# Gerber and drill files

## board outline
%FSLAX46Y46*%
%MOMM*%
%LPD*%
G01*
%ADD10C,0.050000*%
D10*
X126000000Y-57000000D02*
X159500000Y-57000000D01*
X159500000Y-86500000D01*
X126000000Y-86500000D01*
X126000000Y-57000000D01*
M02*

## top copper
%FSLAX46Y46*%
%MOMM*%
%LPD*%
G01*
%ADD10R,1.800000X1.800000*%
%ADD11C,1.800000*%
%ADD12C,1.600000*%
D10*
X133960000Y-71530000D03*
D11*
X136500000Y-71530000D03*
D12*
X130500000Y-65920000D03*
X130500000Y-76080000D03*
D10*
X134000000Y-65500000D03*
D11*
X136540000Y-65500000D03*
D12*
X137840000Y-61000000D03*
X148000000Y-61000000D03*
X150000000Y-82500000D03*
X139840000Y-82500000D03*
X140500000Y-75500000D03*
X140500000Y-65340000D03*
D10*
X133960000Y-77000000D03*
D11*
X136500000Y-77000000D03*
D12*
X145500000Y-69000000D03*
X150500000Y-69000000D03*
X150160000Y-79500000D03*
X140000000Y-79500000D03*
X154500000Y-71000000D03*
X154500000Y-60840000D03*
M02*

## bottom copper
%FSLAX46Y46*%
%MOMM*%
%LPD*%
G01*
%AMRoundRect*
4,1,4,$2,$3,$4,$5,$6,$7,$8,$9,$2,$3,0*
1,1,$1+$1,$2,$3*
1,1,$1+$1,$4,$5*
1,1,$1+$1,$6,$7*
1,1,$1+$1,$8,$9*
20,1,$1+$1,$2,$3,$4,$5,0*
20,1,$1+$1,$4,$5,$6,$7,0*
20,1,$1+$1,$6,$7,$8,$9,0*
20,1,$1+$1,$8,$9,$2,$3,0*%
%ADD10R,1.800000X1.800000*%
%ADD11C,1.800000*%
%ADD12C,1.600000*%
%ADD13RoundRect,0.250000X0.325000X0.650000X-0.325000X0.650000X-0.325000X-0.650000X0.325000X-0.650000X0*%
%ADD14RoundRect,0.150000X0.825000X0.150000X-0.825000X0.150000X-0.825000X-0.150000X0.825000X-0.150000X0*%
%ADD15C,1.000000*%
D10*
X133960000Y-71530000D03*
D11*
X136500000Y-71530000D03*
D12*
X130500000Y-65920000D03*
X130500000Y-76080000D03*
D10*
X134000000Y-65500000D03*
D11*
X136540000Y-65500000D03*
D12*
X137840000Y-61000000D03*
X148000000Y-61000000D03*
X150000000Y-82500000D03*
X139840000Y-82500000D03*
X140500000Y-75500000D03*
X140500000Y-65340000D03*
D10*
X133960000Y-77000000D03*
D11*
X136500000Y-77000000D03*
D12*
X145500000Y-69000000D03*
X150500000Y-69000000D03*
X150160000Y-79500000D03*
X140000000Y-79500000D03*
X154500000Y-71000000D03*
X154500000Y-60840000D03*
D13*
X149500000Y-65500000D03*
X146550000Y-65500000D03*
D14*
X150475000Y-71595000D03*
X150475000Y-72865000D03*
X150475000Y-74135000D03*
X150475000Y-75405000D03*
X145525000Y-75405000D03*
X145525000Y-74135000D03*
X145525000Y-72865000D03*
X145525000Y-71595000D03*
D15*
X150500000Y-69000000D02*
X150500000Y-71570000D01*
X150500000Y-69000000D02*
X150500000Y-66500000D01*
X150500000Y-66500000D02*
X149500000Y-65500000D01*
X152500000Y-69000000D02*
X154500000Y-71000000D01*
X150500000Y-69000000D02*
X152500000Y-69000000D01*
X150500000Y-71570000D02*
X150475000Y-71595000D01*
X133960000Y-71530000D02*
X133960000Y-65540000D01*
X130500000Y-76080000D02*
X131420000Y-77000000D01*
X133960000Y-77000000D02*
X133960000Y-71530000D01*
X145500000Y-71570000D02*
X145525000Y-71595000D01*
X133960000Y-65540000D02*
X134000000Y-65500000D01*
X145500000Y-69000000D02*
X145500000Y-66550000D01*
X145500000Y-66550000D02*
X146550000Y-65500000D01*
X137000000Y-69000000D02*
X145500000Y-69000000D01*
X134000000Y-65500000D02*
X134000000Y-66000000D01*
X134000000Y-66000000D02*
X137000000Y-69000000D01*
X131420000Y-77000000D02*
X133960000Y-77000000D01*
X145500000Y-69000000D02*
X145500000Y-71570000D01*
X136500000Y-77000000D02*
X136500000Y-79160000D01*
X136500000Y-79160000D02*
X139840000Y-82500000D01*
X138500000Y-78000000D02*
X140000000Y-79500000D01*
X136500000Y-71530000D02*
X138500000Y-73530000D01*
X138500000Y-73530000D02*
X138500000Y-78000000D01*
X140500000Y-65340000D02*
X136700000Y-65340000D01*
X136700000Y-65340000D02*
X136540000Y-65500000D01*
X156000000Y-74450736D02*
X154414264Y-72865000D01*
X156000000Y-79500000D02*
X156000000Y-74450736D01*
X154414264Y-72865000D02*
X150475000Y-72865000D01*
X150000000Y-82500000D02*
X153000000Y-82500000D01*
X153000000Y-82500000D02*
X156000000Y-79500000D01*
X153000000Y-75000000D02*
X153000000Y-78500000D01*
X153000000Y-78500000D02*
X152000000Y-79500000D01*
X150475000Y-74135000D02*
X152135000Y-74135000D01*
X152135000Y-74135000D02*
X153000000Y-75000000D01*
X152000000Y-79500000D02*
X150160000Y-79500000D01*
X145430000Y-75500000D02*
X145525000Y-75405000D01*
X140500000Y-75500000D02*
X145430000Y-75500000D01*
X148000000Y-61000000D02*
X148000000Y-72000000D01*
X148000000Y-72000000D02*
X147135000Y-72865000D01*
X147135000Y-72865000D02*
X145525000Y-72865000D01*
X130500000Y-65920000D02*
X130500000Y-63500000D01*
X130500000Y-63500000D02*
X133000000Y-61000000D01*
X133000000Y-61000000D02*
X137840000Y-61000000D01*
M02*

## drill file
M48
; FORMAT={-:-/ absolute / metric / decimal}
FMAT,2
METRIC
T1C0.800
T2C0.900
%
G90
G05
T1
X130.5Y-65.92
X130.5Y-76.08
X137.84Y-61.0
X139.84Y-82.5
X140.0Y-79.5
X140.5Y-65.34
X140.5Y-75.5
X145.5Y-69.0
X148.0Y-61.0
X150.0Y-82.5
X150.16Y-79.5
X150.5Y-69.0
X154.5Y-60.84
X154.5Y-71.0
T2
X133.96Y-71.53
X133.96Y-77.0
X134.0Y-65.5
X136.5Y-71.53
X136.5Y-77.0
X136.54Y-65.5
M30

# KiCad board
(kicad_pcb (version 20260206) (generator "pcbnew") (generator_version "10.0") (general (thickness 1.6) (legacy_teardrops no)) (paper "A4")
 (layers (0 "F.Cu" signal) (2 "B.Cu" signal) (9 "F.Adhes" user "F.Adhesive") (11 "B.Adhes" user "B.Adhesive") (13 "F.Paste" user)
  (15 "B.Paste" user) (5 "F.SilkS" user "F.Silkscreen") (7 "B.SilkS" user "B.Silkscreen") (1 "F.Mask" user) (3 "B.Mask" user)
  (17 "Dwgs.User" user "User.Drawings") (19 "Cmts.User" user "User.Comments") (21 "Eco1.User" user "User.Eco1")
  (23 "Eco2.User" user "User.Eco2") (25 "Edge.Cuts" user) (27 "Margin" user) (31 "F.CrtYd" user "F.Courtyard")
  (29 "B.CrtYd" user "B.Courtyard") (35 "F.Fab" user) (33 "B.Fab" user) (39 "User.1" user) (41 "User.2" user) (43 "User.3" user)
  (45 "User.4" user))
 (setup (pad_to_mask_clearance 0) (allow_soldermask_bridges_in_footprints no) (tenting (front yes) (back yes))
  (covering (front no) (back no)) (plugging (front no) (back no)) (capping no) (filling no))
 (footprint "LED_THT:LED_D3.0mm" (layer "F.Cu") (at 133.96 71.53)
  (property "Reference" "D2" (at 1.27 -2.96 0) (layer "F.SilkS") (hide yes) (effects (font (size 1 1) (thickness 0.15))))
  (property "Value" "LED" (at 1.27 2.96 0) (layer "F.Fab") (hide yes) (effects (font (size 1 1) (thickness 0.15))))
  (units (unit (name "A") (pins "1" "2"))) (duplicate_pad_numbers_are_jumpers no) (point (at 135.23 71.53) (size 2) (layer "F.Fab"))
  (pad "1" thru_hole rect (at 0 0) (size 1.8 1.8) (drill 0.9) (layers "*.Cu" "*.Mask") (remove_unused_layers no) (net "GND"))
  (pad "2" thru_hole circle (at 2.54 0) (size 1.8 1.8) (drill 0.9) (layers "*.Cu" "*.Mask") (remove_unused_layers no) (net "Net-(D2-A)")))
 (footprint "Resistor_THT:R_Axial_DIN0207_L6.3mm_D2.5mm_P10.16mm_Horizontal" (layer "F.Cu") (at 130.5 65.92 -90)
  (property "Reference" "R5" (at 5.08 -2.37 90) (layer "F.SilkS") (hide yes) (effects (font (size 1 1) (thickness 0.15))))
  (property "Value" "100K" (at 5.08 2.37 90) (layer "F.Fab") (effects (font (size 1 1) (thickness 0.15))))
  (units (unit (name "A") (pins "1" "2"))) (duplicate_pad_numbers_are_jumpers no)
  (pad "1" thru_hole circle (at 0 0 270) (size 1.6 1.6) (drill 0.8) (layers "*.Cu" "*.Mask") (remove_unused_layers no)
   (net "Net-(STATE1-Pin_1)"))
  (pad "2" thru_hole circle (at 10.16 0 270) (size 1.6 1.6) (drill 0.8) (layers "*.Cu" "*.Mask") (remove_unused_layers no) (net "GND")))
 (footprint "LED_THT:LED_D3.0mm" (layer "F.Cu") (at 134 65.5)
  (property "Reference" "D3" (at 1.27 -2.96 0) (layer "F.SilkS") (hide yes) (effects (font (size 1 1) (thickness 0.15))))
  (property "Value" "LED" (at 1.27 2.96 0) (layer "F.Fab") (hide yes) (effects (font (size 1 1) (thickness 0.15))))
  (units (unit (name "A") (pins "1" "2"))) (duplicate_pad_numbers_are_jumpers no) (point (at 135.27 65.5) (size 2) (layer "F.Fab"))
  (pad "1" thru_hole rect (at 0 0) (size 1.8 1.8) (drill 0.9) (layers "*.Cu" "*.Mask") (remove_unused_layers no) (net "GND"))
  (pad "2" thru_hole circle (at 2.54 0) (size 1.8 1.8) (drill 0.9) (layers "*.Cu" "*.Mask") (remove_unused_layers no) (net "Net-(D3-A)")))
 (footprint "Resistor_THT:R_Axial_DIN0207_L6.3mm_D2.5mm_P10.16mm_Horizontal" (layer "F.Cu") (at 137.84 61)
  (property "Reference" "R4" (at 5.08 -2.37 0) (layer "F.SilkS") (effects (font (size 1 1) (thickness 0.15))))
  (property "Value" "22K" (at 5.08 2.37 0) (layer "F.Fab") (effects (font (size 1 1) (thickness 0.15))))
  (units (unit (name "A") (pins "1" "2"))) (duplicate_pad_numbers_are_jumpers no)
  (pad "1" thru_hole circle (at 0 0) (size 1.6 1.6) (drill 0.8) (layers "*.Cu" "*.Mask") (remove_unused_layers no)
   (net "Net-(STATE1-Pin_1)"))
  (pad "2" thru_hole circle (at 10.16 0) (size 1.6 1.6) (drill 0.8) (layers "*.Cu" "*.Mask") (remove_unused_layers no) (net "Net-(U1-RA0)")))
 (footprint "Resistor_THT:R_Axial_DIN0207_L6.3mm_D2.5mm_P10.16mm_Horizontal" (layer "F.Cu") (at 150 82.5 180)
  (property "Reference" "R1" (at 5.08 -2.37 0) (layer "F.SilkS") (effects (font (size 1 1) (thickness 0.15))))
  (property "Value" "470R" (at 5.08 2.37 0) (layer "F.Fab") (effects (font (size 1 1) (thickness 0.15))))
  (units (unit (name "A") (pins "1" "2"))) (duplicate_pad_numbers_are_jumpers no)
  (pad "1" thru_hole circle (at 0 0 180) (size 1.6 1.6) (drill 0.8) (layers "*.Cu" "*.Mask") (remove_unused_layers no) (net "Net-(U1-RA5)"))
  (pad "2" thru_hole circle (at 10.16 0 180) (size 1.6 1.6) (drill 0.8) (layers "*.Cu" "*.Mask") (remove_unused_layers no)
   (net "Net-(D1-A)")))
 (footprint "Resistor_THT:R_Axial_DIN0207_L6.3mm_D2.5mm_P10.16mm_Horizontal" (layer "F.Cu") (at 140.5 75.5 90)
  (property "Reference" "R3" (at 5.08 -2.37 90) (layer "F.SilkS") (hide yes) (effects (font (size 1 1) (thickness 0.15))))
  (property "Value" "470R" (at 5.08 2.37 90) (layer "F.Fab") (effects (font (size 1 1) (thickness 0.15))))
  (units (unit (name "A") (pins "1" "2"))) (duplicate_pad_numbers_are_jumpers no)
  (pad "1" thru_hole circle (at 0 0 90) (size 1.6 1.6) (drill 0.8) (layers "*.Cu" "*.Mask") (remove_unused_layers no) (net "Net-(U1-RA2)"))
  (pad "2" thru_hole circle (at 10.16 0 90) (size 1.6 1.6) (drill 0.8) (layers "*.Cu" "*.Mask") (remove_unused_layers no) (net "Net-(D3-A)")))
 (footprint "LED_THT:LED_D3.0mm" (layer "F.Cu") (at 133.96 77)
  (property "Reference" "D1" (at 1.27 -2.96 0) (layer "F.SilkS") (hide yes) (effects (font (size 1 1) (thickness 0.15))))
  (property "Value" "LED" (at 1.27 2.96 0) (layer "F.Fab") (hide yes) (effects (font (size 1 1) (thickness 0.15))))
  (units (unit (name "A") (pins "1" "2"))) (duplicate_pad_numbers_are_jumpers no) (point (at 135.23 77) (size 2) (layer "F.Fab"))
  (pad "1" thru_hole rect (at 0 0) (size 1.8 1.8) (drill 0.9) (layers "*.Cu" "*.Mask") (remove_unused_layers no) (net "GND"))
  (pad "2" thru_hole circle (at 2.54 0) (size 1.8 1.8) (drill 0.9) (layers "*.Cu" "*.Mask") (remove_unused_layers no) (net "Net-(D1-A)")))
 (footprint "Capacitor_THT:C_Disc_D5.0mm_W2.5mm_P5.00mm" (layer "F.Cu") (at 145.5 69)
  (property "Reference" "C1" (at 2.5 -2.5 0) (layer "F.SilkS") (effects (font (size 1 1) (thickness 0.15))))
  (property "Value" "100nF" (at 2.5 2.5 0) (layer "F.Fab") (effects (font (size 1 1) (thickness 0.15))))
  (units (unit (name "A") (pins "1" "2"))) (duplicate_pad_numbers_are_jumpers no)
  (pad "1" thru_hole circle (at 0 0) (size 1.6 1.6) (drill 0.8) (layers "*.Cu" "*.Mask") (remove_unused_layers no) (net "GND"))
  (pad "2" thru_hole circle (at 5 0) (size 1.6 1.6) (drill 0.8) (layers "*.Cu" "*.Mask") (remove_unused_layers no) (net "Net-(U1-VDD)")))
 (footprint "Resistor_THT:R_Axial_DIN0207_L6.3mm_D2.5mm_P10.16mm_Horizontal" (layer "F.Cu") (at 150.16 79.5 180)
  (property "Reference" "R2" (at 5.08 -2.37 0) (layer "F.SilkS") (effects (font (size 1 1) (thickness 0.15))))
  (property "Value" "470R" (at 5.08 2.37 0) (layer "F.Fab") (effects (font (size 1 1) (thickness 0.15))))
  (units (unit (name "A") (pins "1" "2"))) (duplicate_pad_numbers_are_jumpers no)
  (pad "1" thru_hole circle (at 0 0 180) (size 1.6 1.6) (drill 0.8) (layers "*.Cu" "*.Mask") (remove_unused_layers no) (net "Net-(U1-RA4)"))
  (pad "2" thru_hole circle (at 10.16 0 180) (size 1.6 1.6) (drill 0.8) (layers "*.Cu" "*.Mask") (remove_unused_layers no)
   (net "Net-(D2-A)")))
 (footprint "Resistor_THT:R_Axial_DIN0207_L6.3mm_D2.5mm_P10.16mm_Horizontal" (layer "F.Cu") (at 154.5 71 90)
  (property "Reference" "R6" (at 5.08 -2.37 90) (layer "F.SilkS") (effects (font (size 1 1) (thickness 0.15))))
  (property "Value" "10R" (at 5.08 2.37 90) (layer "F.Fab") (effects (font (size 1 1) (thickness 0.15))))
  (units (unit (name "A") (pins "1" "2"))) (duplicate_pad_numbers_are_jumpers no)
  (pad "1" thru_hole circle (at 0 0 90) (size 1.6 1.6) (drill 0.8) (layers "*.Cu" "*.Mask") (remove_unused_layers no) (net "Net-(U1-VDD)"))
  (pad "2" thru_hole circle (at 10.16 0 90) (size 1.6 1.6) (drill 0.8) (layers "*.Cu" "*.Mask") (remove_unused_layers no) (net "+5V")))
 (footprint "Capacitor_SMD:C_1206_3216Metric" (layer "B.Cu") (at 148.025 65.5 180)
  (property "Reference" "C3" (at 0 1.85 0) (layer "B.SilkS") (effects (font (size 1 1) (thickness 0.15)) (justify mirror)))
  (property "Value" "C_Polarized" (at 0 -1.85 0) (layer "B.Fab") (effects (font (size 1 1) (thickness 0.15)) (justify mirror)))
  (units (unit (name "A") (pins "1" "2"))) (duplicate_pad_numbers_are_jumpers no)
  (pad "1" smd roundrect (at -1.475 0 180) (size 1.15 1.8) (layers "B.Cu" "B.Mask" "B.Paste") (roundrect_rratio 0.217391)
   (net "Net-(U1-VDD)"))
  (pad "2" smd roundrect (at 1.475 0 180) (size 1.15 1.8) (layers "B.Cu" "B.Mask" "B.Paste") (roundrect_rratio 0.217391) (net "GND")))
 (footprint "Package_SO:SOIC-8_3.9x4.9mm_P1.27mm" (layer "B.Cu") (at 148 73.5 180)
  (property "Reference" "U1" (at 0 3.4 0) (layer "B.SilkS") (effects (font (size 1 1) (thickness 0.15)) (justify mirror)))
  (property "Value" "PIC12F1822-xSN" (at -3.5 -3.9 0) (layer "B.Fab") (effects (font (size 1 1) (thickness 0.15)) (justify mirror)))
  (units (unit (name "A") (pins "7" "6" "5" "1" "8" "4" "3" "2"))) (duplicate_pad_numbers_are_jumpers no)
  (pad "1" smd roundrect (at -2.475 1.905 180) (size 1.95 0.6) (layers "B.Cu" "B.Mask" "B.Paste") (roundrect_rratio 0.25)
   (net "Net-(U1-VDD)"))
  (pad "2" smd roundrect (at -2.475 0.635 180) (size 1.95 0.6) (layers "B.Cu" "B.Mask" "B.Paste") (roundrect_rratio 0.25)
   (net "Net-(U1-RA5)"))
  (pad "3" smd roundrect (at -2.475 -0.635 180) (size 1.95 0.6) (layers "B.Cu" "B.Mask" "B.Paste") (roundrect_rratio 0.25)
   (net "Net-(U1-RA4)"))
  (pad "4" smd roundrect (at -2.475 -1.905 180) (size 1.95 0.6) (layers "B.Cu" "B.Mask" "B.Paste") (roundrect_rratio 0.25)
   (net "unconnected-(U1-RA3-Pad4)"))
  (pad "5" smd roundrect (at 2.475 -1.905 180) (size 1.95 0.6) (layers "B.Cu" "B.Mask" "B.Paste") (roundrect_rratio 0.25)
   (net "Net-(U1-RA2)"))
  (pad "6" smd roundrect (at 2.475 -0.635 180) (size 1.95 0.6) (layers "B.Cu" "B.Mask" "B.Paste") (roundrect_rratio 0.25)
   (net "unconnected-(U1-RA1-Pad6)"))
  (pad "7" smd roundrect (at 2.475 0.635 180) (size 1.95 0.6) (layers "B.Cu" "B.Mask" "B.Paste") (roundrect_rratio 0.25)
   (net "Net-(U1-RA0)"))
  (pad "8" smd roundrect (at 2.475 1.905 180) (size 1.95 0.6) (layers "B.Cu" "B.Mask" "B.Paste") (roundrect_rratio 0.25) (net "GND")))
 (gr_rect (start 126 57) (end 159.5 86.5) (stroke (width 0.05) (type default)) (fill no) (layer "Edge.Cuts"))
 (segment (start 150.5 69) (end 150.5 71.57) (width 1) (layer "B.Cu") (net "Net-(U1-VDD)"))
 (segment (start 150.5 69) (end 150.5 66.5) (width 1) (layer "B.Cu") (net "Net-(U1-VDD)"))
 (segment (start 150.5 66.5) (end 149.5 65.5) (width 1) (layer "B.Cu") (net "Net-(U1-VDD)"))
 (segment (start 152.5 69) (end 154.5 71) (width 1) (layer "B.Cu") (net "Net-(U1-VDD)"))
 (segment (start 150.5 69) (end 152.5 69) (width 1) (layer "B.Cu") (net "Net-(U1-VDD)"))
 (segment (start 150.5 71.57) (end 150.475 71.595) (width 1) (layer "B.Cu") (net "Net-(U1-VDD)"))
 (segment (start 133.96 71.53) (end 133.96 65.54) (width 1) (layer "B.Cu") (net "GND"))
 (segment (start 130.5 76.08) (end 131.42 77) (width 1) (layer "B.Cu") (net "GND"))
 (segment (start 133.96 77) (end 133.96 71.53) (width 1) (layer "B.Cu") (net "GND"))
 (segment (start 145.5 71.57) (end 145.525 71.595) (width 1) (layer "B.Cu") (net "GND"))
 (segment (start 133.96 65.54) (end 134 65.5) (width 1) (layer "B.Cu") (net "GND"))
 (segment (start 145.5 69) (end 145.5 66.55) (width 1) (layer "B.Cu") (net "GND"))
 (segment (start 145.5 66.55) (end 146.55 65.5) (width 1) (layer "B.Cu") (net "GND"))
 (segment (start 137 69) (end 145.5 69) (width 1) (layer "B.Cu") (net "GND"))
 (segment (start 134 65.5) (end 134 66) (width 1) (layer "B.Cu") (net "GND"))
 (segment (start 134 66) (end 137 69) (width 1) (layer "B.Cu") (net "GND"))
 (segment (start 131.42 77) (end 133.96 77) (width 1) (layer "B.Cu") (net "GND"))
 (segment (start 145.5 69) (end 145.5 71.57) (width 1) (layer "B.Cu") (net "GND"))
 (segment (start 136.5 77) (end 136.5 79.16) (width 1) (layer "B.Cu") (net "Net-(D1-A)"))
 (segment (start 136.5 79.16) (end 139.84 82.5) (width 1) (layer "B.Cu") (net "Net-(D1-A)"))
 (segment (start 138.5 78) (end 140 79.5) (width 1) (layer "B.Cu") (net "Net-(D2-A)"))
 (segment (start 136.5 71.53) (end 138.5 73.53) (width 1) (layer "B.Cu") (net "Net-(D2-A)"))
 (segment (start 138.5 73.53) (end 138.5 78) (width 1) (layer "B.Cu") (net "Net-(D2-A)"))
 (segment (start 140.5 65.34) (end 136.7 65.34) (width 1) (layer "B.Cu") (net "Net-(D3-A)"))
 (segment (start 136.7 65.34) (end 136.54 65.5) (width 1) (layer "B.Cu") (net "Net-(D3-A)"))
 (segment (start 156 74.450736) (end 154.414264 72.865) (width 1) (layer "B.Cu") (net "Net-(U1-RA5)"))
 (segment (start 156 79.5) (end 156 74.450736) (width 1) (layer "B.Cu") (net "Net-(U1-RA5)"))
 (segment (start 154.414264 72.865) (end 150.475 72.865) (width 1) (layer "B.Cu") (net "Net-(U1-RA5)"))
 (segment (start 150 82.5) (end 153 82.5) (width 1) (layer "B.Cu") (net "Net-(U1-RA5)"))
 (segment (start 153 82.5) (end 156 79.5) (width 1) (layer "B.Cu") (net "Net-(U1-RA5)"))
 (segment (start 153 75) (end 153 78.5) (width 1) (layer "B.Cu") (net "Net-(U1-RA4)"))
 (segment (start 153 78.5) (end 152 79.5) (width 1) (layer "B.Cu") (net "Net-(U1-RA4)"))
 (segment (start 150.475 74.135) (end 152.135 74.135) (width 1) (layer "B.Cu") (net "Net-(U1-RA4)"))
 (segment (start 152.135 74.135) (end 153 75) (width 1) (layer "B.Cu") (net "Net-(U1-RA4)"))
 (segment (start 152 79.5) (end 150.16 79.5) (width 1) (layer "B.Cu") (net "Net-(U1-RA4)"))
 (segment (start 145.43 75.5) (end 145.525 75.405) (width 1) (layer "B.Cu") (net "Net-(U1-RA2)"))
 (segment (start 140.5 75.5) (end 145.43 75.5) (width 1) (layer "B.Cu") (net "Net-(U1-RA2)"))
 (segment (start 148 61) (end 148 72) (width 1) (layer "B.Cu") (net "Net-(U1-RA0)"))
 (segment (start 148 72) (end 147.135 72.865) (width 1) (layer "B.Cu") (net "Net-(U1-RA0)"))
 (segment (start 147.135 72.865) (end 145.525 72.865) (width 1) (layer "B.Cu") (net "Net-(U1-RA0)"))
 (segment (start 130.5 65.92) (end 130.5 63.5) (width 1) (layer "B.Cu") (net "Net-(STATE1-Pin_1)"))
 (segment (start 130.5 63.5) (end 133 61) (width 1) (layer "B.Cu") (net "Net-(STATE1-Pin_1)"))
 (segment (start 133 61) (end 137.84 61) (width 1) (layer "B.Cu") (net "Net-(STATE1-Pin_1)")))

